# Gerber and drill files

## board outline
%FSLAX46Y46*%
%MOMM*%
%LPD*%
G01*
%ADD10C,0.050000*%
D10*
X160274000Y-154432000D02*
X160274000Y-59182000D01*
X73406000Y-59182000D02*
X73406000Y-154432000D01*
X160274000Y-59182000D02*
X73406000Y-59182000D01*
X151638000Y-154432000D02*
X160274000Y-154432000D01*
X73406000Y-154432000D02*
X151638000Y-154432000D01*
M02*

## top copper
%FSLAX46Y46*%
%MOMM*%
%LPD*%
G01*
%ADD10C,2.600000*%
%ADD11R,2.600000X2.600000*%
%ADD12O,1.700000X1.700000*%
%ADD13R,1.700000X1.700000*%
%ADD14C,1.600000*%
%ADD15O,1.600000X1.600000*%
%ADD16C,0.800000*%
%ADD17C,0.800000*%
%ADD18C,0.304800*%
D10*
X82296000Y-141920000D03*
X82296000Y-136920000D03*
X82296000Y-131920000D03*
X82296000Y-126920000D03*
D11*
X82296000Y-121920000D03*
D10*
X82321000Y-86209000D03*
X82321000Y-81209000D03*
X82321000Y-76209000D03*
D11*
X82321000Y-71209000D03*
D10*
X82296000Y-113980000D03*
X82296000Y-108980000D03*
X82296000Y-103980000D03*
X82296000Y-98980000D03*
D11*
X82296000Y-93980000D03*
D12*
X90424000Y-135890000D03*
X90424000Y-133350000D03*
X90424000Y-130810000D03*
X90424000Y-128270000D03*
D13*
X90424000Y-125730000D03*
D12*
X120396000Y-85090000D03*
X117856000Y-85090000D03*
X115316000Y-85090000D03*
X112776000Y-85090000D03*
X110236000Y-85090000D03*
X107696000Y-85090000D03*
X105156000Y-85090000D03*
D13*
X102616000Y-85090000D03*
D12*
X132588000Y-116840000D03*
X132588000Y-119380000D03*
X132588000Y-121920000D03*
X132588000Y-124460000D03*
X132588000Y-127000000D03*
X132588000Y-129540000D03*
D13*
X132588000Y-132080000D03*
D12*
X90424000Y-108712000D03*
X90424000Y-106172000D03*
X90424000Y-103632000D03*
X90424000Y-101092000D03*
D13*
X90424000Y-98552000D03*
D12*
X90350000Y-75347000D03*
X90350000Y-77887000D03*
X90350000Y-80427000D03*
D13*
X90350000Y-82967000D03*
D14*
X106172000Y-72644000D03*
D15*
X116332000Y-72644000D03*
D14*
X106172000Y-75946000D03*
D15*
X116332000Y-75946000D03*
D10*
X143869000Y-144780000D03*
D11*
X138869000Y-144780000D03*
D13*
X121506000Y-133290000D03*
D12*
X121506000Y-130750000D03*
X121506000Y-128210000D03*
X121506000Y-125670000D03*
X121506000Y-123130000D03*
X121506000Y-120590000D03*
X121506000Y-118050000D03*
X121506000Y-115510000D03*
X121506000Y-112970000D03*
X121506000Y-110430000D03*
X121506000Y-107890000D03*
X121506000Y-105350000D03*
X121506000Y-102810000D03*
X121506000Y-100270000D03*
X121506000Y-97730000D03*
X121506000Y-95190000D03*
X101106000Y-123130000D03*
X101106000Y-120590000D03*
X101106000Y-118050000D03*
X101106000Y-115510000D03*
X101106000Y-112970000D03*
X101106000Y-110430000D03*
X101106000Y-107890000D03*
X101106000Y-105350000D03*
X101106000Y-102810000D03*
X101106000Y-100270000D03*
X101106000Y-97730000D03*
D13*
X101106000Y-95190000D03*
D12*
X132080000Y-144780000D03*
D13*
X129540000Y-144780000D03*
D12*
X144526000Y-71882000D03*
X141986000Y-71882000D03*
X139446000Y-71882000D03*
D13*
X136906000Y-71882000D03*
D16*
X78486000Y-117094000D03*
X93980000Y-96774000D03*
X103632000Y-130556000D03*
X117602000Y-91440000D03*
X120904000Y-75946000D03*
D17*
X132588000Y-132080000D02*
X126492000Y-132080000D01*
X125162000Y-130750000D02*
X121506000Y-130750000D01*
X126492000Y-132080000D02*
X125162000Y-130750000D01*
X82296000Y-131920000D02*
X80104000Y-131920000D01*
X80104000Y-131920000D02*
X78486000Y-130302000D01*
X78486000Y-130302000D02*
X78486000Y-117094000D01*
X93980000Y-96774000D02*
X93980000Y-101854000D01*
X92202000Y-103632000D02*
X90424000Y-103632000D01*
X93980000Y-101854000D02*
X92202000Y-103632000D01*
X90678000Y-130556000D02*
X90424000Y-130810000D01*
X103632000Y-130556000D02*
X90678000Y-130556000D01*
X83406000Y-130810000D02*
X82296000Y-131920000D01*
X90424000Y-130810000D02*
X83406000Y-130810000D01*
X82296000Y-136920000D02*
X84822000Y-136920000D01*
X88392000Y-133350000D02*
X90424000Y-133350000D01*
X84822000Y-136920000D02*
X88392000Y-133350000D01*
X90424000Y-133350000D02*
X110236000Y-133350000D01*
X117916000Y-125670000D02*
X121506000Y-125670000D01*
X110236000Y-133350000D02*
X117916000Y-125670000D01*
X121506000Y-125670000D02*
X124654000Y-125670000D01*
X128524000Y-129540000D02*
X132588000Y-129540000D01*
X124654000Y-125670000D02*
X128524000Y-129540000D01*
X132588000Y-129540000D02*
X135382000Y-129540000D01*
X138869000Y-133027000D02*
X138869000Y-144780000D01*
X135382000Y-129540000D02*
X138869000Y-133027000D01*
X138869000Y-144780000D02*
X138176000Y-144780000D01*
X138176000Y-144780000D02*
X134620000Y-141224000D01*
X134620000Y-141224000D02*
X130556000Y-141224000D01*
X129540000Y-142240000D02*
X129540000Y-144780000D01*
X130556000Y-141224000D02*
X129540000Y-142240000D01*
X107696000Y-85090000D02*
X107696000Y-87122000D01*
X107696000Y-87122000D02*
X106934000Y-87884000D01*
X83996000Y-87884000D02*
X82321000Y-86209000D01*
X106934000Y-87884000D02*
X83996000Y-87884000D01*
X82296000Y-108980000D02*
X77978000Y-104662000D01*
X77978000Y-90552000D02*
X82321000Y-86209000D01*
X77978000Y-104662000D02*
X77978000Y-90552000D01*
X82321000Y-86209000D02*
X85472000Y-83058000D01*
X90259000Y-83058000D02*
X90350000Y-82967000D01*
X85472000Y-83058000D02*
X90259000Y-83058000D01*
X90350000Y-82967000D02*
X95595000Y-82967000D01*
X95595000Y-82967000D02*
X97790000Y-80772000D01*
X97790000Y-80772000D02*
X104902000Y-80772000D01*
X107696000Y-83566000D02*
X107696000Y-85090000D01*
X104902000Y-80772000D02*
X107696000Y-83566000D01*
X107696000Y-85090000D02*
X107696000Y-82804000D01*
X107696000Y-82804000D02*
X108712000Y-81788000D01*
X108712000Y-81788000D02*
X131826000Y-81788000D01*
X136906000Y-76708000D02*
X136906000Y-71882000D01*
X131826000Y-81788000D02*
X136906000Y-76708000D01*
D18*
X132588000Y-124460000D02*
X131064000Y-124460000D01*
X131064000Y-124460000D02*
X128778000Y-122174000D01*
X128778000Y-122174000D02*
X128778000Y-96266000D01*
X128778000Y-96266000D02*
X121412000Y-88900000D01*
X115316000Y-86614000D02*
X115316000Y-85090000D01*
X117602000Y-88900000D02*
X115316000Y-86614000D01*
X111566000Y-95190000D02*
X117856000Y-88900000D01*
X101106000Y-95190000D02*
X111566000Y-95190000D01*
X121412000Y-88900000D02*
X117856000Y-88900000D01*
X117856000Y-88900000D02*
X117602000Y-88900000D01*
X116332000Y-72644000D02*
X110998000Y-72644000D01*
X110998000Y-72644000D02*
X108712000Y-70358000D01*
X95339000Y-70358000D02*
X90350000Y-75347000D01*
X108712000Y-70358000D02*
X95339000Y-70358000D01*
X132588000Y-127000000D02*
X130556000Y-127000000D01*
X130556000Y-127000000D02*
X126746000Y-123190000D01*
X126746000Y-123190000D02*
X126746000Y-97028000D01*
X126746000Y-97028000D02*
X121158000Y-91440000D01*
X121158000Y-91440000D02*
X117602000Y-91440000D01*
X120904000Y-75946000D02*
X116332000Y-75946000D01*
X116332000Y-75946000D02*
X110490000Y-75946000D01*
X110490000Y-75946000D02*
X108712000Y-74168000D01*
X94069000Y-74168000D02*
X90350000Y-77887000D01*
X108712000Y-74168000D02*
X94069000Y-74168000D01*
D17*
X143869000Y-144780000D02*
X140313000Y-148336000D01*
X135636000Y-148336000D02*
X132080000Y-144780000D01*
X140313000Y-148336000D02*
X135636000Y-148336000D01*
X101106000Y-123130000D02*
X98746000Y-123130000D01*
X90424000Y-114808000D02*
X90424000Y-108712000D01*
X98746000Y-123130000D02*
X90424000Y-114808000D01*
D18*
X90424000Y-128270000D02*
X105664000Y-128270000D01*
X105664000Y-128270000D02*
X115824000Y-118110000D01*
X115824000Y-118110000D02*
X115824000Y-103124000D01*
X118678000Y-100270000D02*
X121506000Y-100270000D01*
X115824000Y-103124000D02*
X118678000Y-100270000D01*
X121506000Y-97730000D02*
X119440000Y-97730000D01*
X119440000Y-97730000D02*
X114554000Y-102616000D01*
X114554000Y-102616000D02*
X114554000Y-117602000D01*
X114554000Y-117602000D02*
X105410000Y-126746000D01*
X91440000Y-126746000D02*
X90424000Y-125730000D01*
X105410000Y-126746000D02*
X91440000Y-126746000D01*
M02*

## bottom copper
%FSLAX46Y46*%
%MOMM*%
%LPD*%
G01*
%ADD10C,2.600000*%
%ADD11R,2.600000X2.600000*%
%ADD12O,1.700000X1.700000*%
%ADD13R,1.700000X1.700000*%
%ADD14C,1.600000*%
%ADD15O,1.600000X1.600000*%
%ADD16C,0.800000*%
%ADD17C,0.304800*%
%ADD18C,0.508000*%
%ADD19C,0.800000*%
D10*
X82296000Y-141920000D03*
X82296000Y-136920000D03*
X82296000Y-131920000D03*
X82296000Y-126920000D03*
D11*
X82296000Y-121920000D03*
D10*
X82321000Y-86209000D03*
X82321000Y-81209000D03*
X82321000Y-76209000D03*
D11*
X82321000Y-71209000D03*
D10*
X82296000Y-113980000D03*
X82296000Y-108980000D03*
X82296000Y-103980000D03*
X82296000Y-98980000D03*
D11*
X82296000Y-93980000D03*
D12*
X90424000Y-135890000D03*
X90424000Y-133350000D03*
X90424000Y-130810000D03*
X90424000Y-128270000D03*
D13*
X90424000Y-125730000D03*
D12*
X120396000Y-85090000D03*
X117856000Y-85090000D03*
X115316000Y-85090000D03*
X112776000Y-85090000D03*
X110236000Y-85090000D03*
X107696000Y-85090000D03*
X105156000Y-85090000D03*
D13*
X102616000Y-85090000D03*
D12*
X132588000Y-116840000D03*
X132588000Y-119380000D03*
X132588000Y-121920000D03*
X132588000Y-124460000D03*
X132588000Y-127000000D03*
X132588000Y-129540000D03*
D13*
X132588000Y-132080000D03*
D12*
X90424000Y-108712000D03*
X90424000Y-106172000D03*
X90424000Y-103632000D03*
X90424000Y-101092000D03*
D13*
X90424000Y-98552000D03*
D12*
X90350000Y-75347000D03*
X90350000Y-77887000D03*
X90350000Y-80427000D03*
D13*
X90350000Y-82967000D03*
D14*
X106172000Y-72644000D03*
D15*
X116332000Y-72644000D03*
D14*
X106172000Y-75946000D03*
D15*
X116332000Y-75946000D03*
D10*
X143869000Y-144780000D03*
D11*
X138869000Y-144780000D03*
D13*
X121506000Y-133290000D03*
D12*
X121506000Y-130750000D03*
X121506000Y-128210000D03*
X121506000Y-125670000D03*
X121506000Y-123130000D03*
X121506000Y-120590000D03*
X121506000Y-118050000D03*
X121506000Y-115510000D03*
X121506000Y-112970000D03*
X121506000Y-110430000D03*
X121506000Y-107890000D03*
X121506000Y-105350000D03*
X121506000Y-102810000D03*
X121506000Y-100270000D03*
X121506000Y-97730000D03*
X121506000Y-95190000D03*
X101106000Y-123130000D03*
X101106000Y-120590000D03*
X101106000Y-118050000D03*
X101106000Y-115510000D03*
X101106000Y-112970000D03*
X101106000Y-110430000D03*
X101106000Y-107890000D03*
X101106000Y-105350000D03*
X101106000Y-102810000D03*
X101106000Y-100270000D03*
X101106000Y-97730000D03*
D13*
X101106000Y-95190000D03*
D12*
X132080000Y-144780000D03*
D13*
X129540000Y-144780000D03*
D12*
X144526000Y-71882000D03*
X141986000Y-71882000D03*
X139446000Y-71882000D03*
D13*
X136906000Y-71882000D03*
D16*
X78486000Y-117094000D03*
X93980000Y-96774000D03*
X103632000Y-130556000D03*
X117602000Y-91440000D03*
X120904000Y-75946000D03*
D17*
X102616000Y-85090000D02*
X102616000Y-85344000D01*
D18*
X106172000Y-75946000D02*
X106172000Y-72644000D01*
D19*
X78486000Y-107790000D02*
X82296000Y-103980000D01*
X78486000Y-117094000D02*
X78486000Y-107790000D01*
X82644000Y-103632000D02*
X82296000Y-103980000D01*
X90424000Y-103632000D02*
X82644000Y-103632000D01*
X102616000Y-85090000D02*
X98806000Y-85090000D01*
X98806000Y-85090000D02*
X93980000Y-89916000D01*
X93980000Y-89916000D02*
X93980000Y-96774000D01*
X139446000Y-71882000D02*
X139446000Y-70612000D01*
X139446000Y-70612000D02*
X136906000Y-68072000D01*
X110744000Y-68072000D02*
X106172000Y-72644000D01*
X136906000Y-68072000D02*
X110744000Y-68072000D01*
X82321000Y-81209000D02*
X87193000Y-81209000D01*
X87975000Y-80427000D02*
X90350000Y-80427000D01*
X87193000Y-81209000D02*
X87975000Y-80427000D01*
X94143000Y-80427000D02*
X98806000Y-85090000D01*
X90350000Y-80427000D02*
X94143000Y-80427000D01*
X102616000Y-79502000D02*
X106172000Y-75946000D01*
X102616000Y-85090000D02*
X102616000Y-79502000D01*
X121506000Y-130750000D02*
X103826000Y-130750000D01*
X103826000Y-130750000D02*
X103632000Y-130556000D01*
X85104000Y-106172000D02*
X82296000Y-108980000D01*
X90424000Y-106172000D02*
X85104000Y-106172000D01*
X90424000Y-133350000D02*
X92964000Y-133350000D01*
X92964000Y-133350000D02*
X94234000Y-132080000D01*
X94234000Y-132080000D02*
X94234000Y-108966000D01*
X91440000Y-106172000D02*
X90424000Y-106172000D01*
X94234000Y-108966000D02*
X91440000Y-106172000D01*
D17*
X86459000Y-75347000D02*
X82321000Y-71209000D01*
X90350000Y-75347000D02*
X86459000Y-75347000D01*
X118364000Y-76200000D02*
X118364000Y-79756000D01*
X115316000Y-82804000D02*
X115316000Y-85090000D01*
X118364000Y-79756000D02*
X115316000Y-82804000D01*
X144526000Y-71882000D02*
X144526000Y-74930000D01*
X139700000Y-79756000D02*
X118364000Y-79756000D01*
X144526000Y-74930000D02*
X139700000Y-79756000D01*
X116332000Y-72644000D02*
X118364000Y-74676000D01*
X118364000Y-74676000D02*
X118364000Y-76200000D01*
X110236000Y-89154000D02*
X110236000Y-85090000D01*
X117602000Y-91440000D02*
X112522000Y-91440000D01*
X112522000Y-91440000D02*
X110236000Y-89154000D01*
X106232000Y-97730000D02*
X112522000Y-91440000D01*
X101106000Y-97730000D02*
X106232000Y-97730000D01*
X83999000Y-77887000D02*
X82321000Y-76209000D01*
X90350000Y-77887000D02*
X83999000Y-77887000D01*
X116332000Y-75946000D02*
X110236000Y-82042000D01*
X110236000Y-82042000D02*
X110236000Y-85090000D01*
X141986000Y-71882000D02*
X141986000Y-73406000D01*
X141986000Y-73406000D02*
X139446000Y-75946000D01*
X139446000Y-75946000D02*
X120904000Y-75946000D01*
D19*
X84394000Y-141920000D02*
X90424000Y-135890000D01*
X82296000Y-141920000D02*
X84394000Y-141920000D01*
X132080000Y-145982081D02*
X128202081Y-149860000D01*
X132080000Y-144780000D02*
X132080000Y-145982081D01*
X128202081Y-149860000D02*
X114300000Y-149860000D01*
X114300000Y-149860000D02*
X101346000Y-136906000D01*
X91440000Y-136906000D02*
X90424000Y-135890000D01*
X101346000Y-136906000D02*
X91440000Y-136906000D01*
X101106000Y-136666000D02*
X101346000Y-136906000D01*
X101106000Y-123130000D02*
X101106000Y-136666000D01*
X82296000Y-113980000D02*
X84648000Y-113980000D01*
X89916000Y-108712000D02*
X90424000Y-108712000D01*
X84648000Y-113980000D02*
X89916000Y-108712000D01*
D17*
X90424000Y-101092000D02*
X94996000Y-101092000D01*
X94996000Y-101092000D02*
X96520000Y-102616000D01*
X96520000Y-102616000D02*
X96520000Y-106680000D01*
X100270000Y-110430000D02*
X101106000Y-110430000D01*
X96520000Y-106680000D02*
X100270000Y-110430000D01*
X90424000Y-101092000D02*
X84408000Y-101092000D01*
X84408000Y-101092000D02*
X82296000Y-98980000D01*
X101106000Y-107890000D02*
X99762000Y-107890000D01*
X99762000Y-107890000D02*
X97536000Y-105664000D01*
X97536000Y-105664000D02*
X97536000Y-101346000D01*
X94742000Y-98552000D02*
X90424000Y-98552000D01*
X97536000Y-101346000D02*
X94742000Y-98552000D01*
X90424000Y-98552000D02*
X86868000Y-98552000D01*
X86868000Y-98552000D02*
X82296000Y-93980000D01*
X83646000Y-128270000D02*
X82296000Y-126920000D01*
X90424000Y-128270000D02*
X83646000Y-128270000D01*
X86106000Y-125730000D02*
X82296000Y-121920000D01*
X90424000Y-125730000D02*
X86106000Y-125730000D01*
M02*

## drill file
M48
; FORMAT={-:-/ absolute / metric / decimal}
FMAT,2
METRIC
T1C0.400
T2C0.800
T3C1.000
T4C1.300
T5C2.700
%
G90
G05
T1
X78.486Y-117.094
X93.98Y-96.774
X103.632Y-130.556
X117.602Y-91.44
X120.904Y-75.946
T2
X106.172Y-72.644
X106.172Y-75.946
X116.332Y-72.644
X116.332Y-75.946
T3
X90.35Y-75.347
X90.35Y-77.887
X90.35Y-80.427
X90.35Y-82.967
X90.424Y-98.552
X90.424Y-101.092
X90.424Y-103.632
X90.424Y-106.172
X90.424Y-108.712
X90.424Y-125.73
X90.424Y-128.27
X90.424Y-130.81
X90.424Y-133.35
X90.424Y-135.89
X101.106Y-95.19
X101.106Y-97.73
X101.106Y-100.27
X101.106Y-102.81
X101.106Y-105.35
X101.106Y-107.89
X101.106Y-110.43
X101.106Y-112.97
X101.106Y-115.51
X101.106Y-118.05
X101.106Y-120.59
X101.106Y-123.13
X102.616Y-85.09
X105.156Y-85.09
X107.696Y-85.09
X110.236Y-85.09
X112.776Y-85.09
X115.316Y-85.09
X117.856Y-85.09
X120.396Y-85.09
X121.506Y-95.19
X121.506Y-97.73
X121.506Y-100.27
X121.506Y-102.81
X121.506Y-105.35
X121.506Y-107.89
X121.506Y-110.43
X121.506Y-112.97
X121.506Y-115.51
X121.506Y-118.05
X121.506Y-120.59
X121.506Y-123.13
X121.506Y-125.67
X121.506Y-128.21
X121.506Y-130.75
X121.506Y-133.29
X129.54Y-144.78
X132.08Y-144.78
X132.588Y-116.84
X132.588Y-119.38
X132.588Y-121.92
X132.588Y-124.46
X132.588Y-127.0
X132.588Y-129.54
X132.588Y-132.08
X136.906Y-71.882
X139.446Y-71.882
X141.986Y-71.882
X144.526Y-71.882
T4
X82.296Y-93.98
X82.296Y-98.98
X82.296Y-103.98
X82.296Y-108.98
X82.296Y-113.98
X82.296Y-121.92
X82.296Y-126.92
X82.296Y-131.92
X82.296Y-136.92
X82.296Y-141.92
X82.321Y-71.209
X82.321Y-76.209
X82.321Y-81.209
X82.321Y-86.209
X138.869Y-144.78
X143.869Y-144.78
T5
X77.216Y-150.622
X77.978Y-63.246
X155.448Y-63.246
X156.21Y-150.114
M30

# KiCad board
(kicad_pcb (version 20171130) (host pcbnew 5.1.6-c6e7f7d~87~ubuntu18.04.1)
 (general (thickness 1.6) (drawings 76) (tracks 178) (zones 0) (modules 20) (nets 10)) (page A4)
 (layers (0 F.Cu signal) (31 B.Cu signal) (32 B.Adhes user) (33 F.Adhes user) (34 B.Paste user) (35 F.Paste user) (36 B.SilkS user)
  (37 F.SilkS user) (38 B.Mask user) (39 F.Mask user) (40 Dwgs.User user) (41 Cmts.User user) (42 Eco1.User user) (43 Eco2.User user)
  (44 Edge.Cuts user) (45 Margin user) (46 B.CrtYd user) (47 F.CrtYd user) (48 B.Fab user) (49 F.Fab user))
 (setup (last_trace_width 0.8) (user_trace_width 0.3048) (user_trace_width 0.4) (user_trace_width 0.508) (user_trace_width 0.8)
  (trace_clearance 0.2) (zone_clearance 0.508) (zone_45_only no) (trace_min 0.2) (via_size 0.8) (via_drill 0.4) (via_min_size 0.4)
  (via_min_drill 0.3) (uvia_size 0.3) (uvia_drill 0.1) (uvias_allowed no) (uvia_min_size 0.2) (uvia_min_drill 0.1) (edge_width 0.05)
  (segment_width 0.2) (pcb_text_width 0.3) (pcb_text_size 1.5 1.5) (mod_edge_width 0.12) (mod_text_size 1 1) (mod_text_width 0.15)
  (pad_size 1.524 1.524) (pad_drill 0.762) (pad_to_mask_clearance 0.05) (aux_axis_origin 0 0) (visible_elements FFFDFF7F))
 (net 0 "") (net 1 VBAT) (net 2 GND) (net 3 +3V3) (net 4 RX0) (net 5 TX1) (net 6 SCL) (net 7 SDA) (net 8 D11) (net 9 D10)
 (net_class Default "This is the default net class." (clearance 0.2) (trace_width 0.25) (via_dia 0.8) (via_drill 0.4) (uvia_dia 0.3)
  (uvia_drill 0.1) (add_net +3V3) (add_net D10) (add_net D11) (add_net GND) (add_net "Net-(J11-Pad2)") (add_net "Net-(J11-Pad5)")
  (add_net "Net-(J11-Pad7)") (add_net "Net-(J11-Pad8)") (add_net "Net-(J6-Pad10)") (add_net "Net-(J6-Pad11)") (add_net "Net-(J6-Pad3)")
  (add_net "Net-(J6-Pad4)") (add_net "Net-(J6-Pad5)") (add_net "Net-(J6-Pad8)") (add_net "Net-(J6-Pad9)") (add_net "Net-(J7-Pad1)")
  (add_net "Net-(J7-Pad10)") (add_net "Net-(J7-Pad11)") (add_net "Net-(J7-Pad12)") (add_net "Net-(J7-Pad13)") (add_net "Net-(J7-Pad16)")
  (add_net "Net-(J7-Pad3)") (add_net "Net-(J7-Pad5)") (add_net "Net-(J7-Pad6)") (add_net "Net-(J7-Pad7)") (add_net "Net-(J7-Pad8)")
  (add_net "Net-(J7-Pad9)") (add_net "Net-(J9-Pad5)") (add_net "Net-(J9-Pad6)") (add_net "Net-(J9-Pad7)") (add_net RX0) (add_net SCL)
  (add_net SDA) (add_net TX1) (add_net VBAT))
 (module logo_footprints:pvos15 (layer F.Cu) (at 89.408 148.844)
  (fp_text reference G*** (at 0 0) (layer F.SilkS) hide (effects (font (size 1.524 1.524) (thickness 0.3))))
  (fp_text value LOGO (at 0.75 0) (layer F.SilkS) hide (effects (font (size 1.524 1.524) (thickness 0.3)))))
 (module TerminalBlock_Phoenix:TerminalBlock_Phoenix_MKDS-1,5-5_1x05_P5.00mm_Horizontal (layer F.Cu) (at 82.296 121.92 270)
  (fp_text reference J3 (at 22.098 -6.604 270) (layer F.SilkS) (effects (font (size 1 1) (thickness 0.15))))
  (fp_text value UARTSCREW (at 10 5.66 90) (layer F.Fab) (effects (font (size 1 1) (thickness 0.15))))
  (pad 5 thru_hole circle (at 20 0 270) (size 2.6 2.6) (drill 1.3) (layers *.Cu *.Mask) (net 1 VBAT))
  (pad 4 thru_hole circle (at 15 0 270) (size 2.6 2.6) (drill 1.3) (layers *.Cu *.Mask) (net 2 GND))
  (pad 3 thru_hole circle (at 10 0 270) (size 2.6 2.6) (drill 1.3) (layers *.Cu *.Mask) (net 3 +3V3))
  (pad 2 thru_hole circle (at 5 0 270) (size 2.6 2.6) (drill 1.3) (layers *.Cu *.Mask) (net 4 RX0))
  (pad 1 thru_hole rect (at 0 0 270) (size 2.6 2.6) (drill 1.3) (layers *.Cu *.Mask) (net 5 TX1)))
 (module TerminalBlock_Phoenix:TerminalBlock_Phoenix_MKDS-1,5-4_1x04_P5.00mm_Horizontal (layer F.Cu) (at 82.321 71.209 270)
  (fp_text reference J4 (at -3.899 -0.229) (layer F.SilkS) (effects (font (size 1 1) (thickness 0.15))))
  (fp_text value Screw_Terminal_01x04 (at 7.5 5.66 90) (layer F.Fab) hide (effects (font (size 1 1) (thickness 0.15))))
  (pad 4 thru_hole circle (at 15 0 270) (size 2.6 2.6) (drill 1.3) (layers *.Cu *.Mask) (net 2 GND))
  (pad 3 thru_hole circle (at 10 0 270) (size 2.6 2.6) (drill 1.3) (layers *.Cu *.Mask) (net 3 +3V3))
  (pad 2 thru_hole circle (at 5 0 270) (size 2.6 2.6) (drill 1.3) (layers *.Cu *.Mask) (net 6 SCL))
  (pad 1 thru_hole rect (at 0 0 270) (size 2.6 2.6) (drill 1.3) (layers *.Cu *.Mask) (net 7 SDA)))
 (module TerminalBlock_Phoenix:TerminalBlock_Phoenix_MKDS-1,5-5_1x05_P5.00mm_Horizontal (layer F.Cu) (at 82.296 93.98 270)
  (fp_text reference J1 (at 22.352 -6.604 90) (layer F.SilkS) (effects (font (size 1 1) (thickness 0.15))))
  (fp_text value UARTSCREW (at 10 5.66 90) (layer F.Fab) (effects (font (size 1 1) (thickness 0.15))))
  (pad 5 thru_hole circle (at 20 0 270) (size 2.6 2.6) (drill 1.3) (layers *.Cu *.Mask) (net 1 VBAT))
  (pad 4 thru_hole circle (at 15 0 270) (size 2.6 2.6) (drill 1.3) (layers *.Cu *.Mask) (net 2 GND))
  (pad 3 thru_hole circle (at 10 0 270) (size 2.6 2.6) (drill 1.3) (layers *.Cu *.Mask) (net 3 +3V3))
  (pad 2 thru_hole circle (at 5 0 270) (size 2.6 2.6) (drill 1.3) (layers *.Cu *.Mask) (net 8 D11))
  (pad 1 thru_hole rect (at 0 0 270) (size 2.6 2.6) (drill 1.3) (layers *.Cu *.Mask) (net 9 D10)))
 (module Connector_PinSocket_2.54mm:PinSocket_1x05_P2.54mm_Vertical (layer F.Cu) (at 90.424 125.73)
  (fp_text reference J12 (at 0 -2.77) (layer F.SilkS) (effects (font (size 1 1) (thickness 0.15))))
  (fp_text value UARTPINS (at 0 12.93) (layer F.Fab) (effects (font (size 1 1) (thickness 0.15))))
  (pad 5 thru_hole oval (at 0 10.16) (size 1.7 1.7) (drill 1) (layers *.Cu *.Mask) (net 1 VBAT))
  (pad 4 thru_hole oval (at 0 7.62) (size 1.7 1.7) (drill 1) (layers *.Cu *.Mask) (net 2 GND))
  (pad 3 thru_hole oval (at 0 5.08) (size 1.7 1.7) (drill 1) (layers *.Cu *.Mask) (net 3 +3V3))
  (pad 2 thru_hole oval (at 0 2.54) (size 1.7 1.7) (drill 1) (layers *.Cu *.Mask) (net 4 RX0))
  (pad 1 thru_hole rect (at 0 0) (size 1.7 1.7) (drill 1) (layers *.Cu *.Mask) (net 5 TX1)))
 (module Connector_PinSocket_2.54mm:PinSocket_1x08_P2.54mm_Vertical (layer F.Cu) (at 102.616 85.09 90)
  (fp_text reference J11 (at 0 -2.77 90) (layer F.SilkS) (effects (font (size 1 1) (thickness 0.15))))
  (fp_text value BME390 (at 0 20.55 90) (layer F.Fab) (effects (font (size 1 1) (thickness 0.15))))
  (pad 8 thru_hole oval (at 0 17.78 90) (size 1.7 1.7) (drill 1) (layers *.Cu *.Mask))
  (pad 7 thru_hole oval (at 0 15.24 90) (size 1.7 1.7) (drill 1) (layers *.Cu *.Mask))
  (pad 6 thru_hole oval (at 0 12.7 90) (size 1.7 1.7) (drill 1) (layers *.Cu *.Mask) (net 7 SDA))
  (pad 5 thru_hole oval (at 0 10.16 90) (size 1.7 1.7) (drill 1) (layers *.Cu *.Mask))
  (pad 4 thru_hole oval (at 0 7.62 90) (size 1.7 1.7) (drill 1) (layers *.Cu *.Mask) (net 6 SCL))
  (pad 3 thru_hole oval (at 0 5.08 90) (size 1.7 1.7) (drill 1) (layers *.Cu *.Mask) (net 2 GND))
  (pad 2 thru_hole oval (at 0 2.54 90) (size 1.7 1.7) (drill 1) (layers *.Cu *.Mask))
  (pad 1 thru_hole rect (at 0 0 90) (size 1.7 1.7) (drill 1) (layers *.Cu *.Mask) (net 3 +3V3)))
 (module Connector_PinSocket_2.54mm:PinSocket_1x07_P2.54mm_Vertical (layer F.Cu) (at 132.588 132.08 180)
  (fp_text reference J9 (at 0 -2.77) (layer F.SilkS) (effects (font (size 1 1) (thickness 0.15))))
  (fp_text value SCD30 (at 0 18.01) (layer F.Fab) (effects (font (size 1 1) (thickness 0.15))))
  (pad 7 thru_hole oval (at 0 15.24 180) (size 1.7 1.7) (drill 1) (layers *.Cu *.Mask))
  (pad 6 thru_hole oval (at 0 12.7 180) (size 1.7 1.7) (drill 1) (layers *.Cu *.Mask))
  (pad 5 thru_hole oval (at 0 10.16 180) (size 1.7 1.7) (drill 1) (layers *.Cu *.Mask))
  (pad 4 thru_hole oval (at 0 7.62 180) (size 1.7 1.7) (drill 1) (layers *.Cu *.Mask) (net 7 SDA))
  (pad 3 thru_hole oval (at 0 5.08 180) (size 1.7 1.7) (drill 1) (layers *.Cu *.Mask) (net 6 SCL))
  (pad 2 thru_hole oval (at 0 2.54 180) (size 1.7 1.7) (drill 1) (layers *.Cu *.Mask) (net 2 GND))
  (pad 1 thru_hole rect (at 0 0 180) (size 1.7 1.7) (drill 1) (layers *.Cu *.Mask) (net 3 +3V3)))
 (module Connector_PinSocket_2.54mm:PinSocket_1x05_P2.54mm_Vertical (layer F.Cu) (at 90.424 98.552)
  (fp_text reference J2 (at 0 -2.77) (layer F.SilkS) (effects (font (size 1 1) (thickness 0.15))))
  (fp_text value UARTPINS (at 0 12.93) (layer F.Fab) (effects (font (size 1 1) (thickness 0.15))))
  (pad 5 thru_hole oval (at 0 10.16) (size 1.7 1.7) (drill 1) (layers *.Cu *.Mask) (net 1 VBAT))
  (pad 4 thru_hole oval (at 0 7.62) (size 1.7 1.7) (drill 1) (layers *.Cu *.Mask) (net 2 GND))
  (pad 3 thru_hole oval (at 0 5.08) (size 1.7 1.7) (drill 1) (layers *.Cu *.Mask) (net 3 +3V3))
  (pad 2 thru_hole oval (at 0 2.54) (size 1.7 1.7) (drill 1) (layers *.Cu *.Mask) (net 8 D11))
  (pad 1 thru_hole rect (at 0 0) (size 1.7 1.7) (drill 1) (layers *.Cu *.Mask) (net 9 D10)))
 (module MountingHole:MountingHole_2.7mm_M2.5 (layer F.Cu) (at 156.21 150.114)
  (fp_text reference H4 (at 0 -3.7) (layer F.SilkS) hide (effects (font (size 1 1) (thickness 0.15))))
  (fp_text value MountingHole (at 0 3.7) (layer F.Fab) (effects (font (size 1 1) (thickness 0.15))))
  (pad 1 np_thru_hole circle (at 0 0) (size 2.7 2.7) (drill 2.7) (layers *.Cu *.Mask)))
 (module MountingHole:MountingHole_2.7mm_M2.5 (layer F.Cu) (at 77.216 150.622)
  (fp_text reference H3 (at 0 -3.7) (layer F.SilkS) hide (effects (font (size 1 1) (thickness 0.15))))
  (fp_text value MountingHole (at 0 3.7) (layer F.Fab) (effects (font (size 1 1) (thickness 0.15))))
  (pad 1 np_thru_hole circle (at 0 0) (size 2.7 2.7) (drill 2.7) (layers *.Cu *.Mask)))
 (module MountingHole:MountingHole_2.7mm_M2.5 (layer F.Cu) (at 155.448 63.246)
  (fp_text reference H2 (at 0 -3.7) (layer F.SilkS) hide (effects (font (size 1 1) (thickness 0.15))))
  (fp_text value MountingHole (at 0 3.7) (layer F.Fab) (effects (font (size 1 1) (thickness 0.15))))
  (pad 1 np_thru_hole circle (at 0 0) (size 2.7 2.7) (drill 2.7) (layers *.Cu *.Mask)))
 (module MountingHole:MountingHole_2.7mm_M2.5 (layer F.Cu) (at 77.978 63.246)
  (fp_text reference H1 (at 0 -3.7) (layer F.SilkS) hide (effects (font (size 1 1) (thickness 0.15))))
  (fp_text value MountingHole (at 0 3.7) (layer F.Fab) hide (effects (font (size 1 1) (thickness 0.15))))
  (pad 1 np_thru_hole circle (at 0 0) (size 2.7 2.7) (drill 2.7) (layers *.Cu *.Mask)))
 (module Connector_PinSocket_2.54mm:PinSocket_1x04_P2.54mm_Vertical (layer F.Cu) (at 90.35 82.967 180)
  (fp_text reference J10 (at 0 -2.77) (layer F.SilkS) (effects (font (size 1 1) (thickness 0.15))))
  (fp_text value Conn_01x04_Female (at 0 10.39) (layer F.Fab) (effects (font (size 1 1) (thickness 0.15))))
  (pad 4 thru_hole oval (at 0 7.62 180) (size 1.7 1.7) (drill 1) (layers *.Cu *.Mask) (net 7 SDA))
  (pad 3 thru_hole oval (at 0 5.08 180) (size 1.7 1.7) (drill 1) (layers *.Cu *.Mask) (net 6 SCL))
  (pad 2 thru_hole oval (at 0 2.54 180) (size 1.7 1.7) (drill 1) (layers *.Cu *.Mask) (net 3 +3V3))
  (pad 1 thru_hole rect (at 0 0 180) (size 1.7 1.7) (drill 1) (layers *.Cu *.Mask) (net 2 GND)))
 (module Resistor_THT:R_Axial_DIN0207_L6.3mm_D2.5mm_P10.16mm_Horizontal (layer F.Cu) (at 106.172 72.644)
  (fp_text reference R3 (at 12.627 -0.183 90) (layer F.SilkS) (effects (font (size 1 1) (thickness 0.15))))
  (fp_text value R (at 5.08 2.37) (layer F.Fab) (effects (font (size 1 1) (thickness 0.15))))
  (pad 1 thru_hole circle (at 0 0) (size 1.6 1.6) (drill 0.8) (layers *.Cu *.Mask) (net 3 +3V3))
  (pad 2 thru_hole oval (at 10.16 0) (size 1.6 1.6) (drill 0.8) (layers *.Cu *.Mask) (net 7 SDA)))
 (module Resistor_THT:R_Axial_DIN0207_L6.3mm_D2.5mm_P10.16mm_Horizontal (layer F.Cu) (at 106.172 75.946)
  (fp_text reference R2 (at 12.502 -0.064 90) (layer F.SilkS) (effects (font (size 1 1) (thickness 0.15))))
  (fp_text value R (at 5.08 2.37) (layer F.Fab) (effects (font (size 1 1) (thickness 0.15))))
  (pad 1 thru_hole circle (at 0 0) (size 1.6 1.6) (drill 0.8) (layers *.Cu *.Mask) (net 3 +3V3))
  (pad 2 thru_hole oval (at 10.16 0) (size 1.6 1.6) (drill 0.8) (layers *.Cu *.Mask) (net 6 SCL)))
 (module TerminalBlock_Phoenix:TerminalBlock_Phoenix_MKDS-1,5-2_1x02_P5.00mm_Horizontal (layer F.Cu) (at 138.869 144.78)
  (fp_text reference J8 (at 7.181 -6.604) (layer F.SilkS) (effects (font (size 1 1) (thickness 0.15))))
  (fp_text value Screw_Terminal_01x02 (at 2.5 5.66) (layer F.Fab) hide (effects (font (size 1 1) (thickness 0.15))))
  (pad 2 thru_hole circle (at 5 0) (size 2.6 2.6) (drill 1.3) (layers *.Cu *.Mask) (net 1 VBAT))
  (pad 1 thru_hole rect (at 0 0) (size 2.6 2.6) (drill 1.3) (layers *.Cu *.Mask) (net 2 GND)))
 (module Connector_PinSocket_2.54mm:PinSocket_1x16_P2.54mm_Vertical (layer F.Cu) (at 121.506 133.29 180)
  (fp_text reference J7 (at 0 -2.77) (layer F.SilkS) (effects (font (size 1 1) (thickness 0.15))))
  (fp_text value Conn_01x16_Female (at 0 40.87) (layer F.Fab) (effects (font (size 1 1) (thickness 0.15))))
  (pad 1 thru_hole rect (at 0 0 180) (size 1.7 1.7) (drill 1) (layers *.Cu *.Mask))
  (pad 2 thru_hole oval (at 0 2.54 180) (size 1.7 1.7) (drill 1) (layers *.Cu *.Mask) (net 3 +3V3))
  (pad 3 thru_hole oval (at 0 5.08 180) (size 1.7 1.7) (drill 1) (layers *.Cu *.Mask))
  (pad 4 thru_hole oval (at 0 7.62 180) (size 1.7 1.7) (drill 1) (layers *.Cu *.Mask) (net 2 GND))
  (pad 5 thru_hole oval (at 0 10.16 180) (size 1.7 1.7) (drill 1) (layers *.Cu *.Mask))
  (pad 6 thru_hole oval (at 0 12.7 180) (size 1.7 1.7) (drill 1) (layers *.Cu *.Mask))
  (pad 7 thru_hole oval (at 0 15.24 180) (size 1.7 1.7) (drill 1) (layers *.Cu *.Mask))
  (pad 8 thru_hole oval (at 0 17.78 180) (size 1.7 1.7) (drill 1) (layers *.Cu *.Mask))
  (pad 9 thru_hole oval (at 0 20.32 180) (size 1.7 1.7) (drill 1) (layers *.Cu *.Mask))
  (pad 10 thru_hole oval (at 0 22.86 180) (size 1.7 1.7) (drill 1) (layers *.Cu *.Mask))
  (pad 11 thru_hole oval (at 0 25.4 180) (size 1.7 1.7) (drill 1) (layers *.Cu *.Mask))
  (pad 12 thru_hole oval (at 0 27.94 180) (size 1.7 1.7) (drill 1) (layers *.Cu *.Mask))
  (pad 13 thru_hole oval (at 0 30.48 180) (size 1.7 1.7) (drill 1) (layers *.Cu *.Mask))
  (pad 14 thru_hole oval (at 0 33.02 180) (size 1.7 1.7) (drill 1) (layers *.Cu *.Mask) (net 4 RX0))
  (pad 15 thru_hole oval (at 0 35.56 180) (size 1.7 1.7) (drill 1) (layers *.Cu *.Mask) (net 5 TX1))
  (pad 16 thru_hole oval (at 0 38.1 180) (size 1.7 1.7) (drill 1) (layers *.Cu *.Mask)))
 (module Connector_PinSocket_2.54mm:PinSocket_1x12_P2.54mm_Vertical (layer F.Cu) (at 101.106 95.19)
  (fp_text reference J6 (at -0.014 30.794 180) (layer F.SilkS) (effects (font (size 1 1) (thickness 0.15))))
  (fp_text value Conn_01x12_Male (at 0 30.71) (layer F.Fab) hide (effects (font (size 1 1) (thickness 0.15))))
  (pad 12 thru_hole oval (at 0 27.94) (size 1.7 1.7) (drill 1) (layers *.Cu *.Mask) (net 1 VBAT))
  (pad 11 thru_hole oval (at 0 25.4) (size 1.7 1.7) (drill 1) (layers *.Cu *.Mask))
  (pad 10 thru_hole oval (at 0 22.86) (size 1.7 1.7) (drill 1) (layers *.Cu *.Mask))
  (pad 9 thru_hole oval (at 0 20.32) (size 1.7 1.7) (drill 1) (layers *.Cu *.Mask))
  (pad 8 thru_hole oval (at 0 17.78) (size 1.7 1.7) (drill 1) (layers *.Cu *.Mask))
  (pad 7 thru_hole oval (at 0 15.24) (size 1.7 1.7) (drill 1) (layers *.Cu *.Mask) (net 8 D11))
  (pad 6 thru_hole oval (at 0 12.7) (size 1.7 1.7) (drill 1) (layers *.Cu *.Mask) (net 9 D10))
  (pad 5 thru_hole oval (at 0 10.16) (size 1.7 1.7) (drill 1) (layers *.Cu *.Mask))
  (pad 4 thru_hole oval (at 0 7.62) (size 1.7 1.7) (drill 1) (layers *.Cu *.Mask))
  (pad 3 thru_hole oval (at 0 5.08) (size 1.7 1.7) (drill 1) (layers *.Cu *.Mask))
  (pad 2 thru_hole oval (at 0 2.54) (size 1.7 1.7) (drill 1) (layers *.Cu *.Mask) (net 6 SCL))
  (pad 1 thru_hole rect (at 0 0) (size 1.7 1.7) (drill 1) (layers *.Cu *.Mask) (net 7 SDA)))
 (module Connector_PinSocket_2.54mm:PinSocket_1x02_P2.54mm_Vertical (layer F.Cu) (at 129.54 144.78 90)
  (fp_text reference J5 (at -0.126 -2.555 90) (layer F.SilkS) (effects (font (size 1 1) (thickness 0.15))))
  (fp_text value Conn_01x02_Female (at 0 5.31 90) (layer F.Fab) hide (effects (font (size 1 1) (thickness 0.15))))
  (pad 2 thru_hole oval (at 0 2.54 90) (size 1.7 1.7) (drill 1) (layers *.Cu *.Mask) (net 1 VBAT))
  (pad 1 thru_hole rect (at 0 0 90) (size 1.7 1.7) (drill 1) (layers *.Cu *.Mask) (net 2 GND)))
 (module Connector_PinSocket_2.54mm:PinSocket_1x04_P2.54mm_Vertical (layer F.Cu) (at 136.906 71.882 90)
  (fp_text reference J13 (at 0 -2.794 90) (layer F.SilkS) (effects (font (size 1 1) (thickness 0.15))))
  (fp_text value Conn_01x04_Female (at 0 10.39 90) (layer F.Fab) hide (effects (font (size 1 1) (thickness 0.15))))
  (pad 4 thru_hole oval (at 0 7.62 90) (size 1.7 1.7) (drill 1) (layers *.Cu *.Mask) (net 7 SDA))
  (pad 3 thru_hole oval (at 0 5.08 90) (size 1.7 1.7) (drill 1) (layers *.Cu *.Mask) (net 6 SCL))
  (pad 2 thru_hole oval (at 0 2.54 90) (size 1.7 1.7) (drill 1) (layers *.Cu *.Mask) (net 3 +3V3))
  (pad 1 thru_hole rect (at 0 0 90) (size 1.7 1.7) (drill 1) (layers *.Cu *.Mask) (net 2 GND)))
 (gr_line (start 160.274 154.432) (end 160.274 59.182) (layer Edge.Cuts) (width 0.05))
 (gr_line (start 73.406 59.182) (end 73.406 154.432) (layer Edge.Cuts) (width 0.05))
 (gr_line (start 160.274 59.182) (end 73.406 59.182) (layer Edge.Cuts) (width 0.05))
 (gr_line (start 151.638 154.432) (end 160.274 154.432) (layer Edge.Cuts) (width 0.05))
 (gr_line (start 73.406 154.432) (end 151.638 154.432) (layer Edge.Cuts) (width 0.05))
 (segment (start 102.616 85.09) (end 102.616 85.344) (width 0.3048) (layer B.Cu) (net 3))
 (segment (start 106.172 75.946) (end 106.172 72.644) (width 0.508) (layer B.Cu) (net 3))
 (segment (start 132.588 132.08) (end 126.492 132.08) (width 0.8) (layer F.Cu) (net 3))
 (segment (start 125.162 130.75) (end 121.506 130.75) (width 0.8) (layer F.Cu) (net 3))
 (segment (start 126.492 132.08) (end 125.162 130.75) (width 0.8) (layer F.Cu) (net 3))
 (segment (start 82.296 131.92) (end 80.104 131.92) (width 0.8) (layer F.Cu) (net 3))
 (segment (start 80.104 131.92) (end 78.486 130.302) (width 0.8) (layer F.Cu) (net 3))
 (via (at 78.486 117.094) (size 0.8) (drill 0.4) (layers F.Cu B.Cu) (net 3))
 (segment (start 78.486 130.302) (end 78.486 117.094) (width 0.8) (layer F.Cu) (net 3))
 (segment (start 78.486 107.79) (end 82.296 103.98) (width 0.8) (layer B.Cu) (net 3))
 (segment (start 78.486 117.094) (end 78.486 107.79) (width 0.8) (layer B.Cu) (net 3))
 (segment (start 82.644 103.632) (end 82.296 103.98) (width 0.8) (layer B.Cu) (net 3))
 (segment (start 90.424 103.632) (end 82.644 103.632) (width 0.8) (layer B.Cu) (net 3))
 (segment (start 102.616 85.09) (end 98.806 85.09) (width 0.8) (layer B.Cu) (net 3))
 (via (at 93.98 96.774) (size 0.8) (drill 0.4) (layers F.Cu B.Cu) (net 3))
 (segment (start 98.806 85.09) (end 93.98 89.916) (width 0.8) (layer B.Cu) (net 3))
 (segment (start 93.98 89.916) (end 93.98 96.774) (width 0.8) (layer B.Cu) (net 3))
 (segment (start 93.98 96.774) (end 93.98 101.854) (width 0.8) (layer F.Cu) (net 3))
 (segment (start 92.202 103.632) (end 90.424 103.632) (width 0.8) (layer F.Cu) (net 3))
 (segment (start 93.98 101.854) (end 92.202 103.632) (width 0.8) (layer F.Cu) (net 3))
 (segment (start 139.446 71.882) (end 139.446 70.612) (width 0.8) (layer B.Cu) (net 3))
 (segment (start 139.446 70.612) (end 136.906 68.072) (width 0.8) (layer B.Cu) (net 3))
 (segment (start 110.744 68.072) (end 106.172 72.644) (width 0.8) (layer B.Cu) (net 3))
 (segment (start 136.906 68.072) (end 110.744 68.072) (width 0.8) (layer B.Cu) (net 3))
 (segment (start 82.321 81.209) (end 87.193 81.209) (width 0.8) (layer B.Cu) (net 3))
 (segment (start 87.975 80.427) (end 90.35 80.427) (width 0.8) (layer B.Cu) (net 3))
 (segment (start 87.193 81.209) (end 87.975 80.427) (width 0.8) (layer B.Cu) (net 3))
 (segment (start 94.143 80.427) (end 98.806 85.09) (width 0.8) (layer B.Cu) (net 3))
 (segment (start 90.35 80.427) (end 94.143 80.427) (width 0.8) (layer B.Cu) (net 3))
 (segment (start 102.616 79.502) (end 106.172 75.946) (width 0.8) (layer B.Cu) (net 3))
 (segment (start 102.616 85.09) (end 102.616 79.502) (width 0.8) (layer B.Cu) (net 3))
 (via (at 103.632 130.556) (size 0.8) (drill 0.4) (layers F.Cu B.Cu) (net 3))
 (segment (start 121.506 130.75) (end 103.826 130.75) (width 0.8) (layer B.Cu) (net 3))
 (segment (start 103.826 130.75) (end 103.632 130.556) (width 0.8) (layer B.Cu) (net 3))
 (segment (start 90.678 130.556) (end 90.424 130.81) (width 0.8) (layer F.Cu) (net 3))
 (segment (start 103.632 130.556) (end 90.678 130.556) (width 0.8) (layer F.Cu) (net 3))
 (segment (start 83.406 130.81) (end 82.296 131.92) (width 0.8) (layer F.Cu) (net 3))
 (segment (start 90.424 130.81) (end 83.406 130.81) (width 0.8) (layer F.Cu) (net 3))
 (segment (start 82.296 136.92) (end 84.822 136.92) (width 0.8) (layer F.Cu) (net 2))
 (segment (start 88.392 133.35) (end 90.424 133.35) (width 0.8) (layer F.Cu) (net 2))
 (segment (start 84.822 136.92) (end 88.392 133.35) (width 0.8) (layer F.Cu) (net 2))
 (segment (start 90.424 133.35) (end 110.236 133.35) (width 0.8) (layer F.Cu) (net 2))
 (segment (start 117.916 125.67) (end 121.506 125.67) (width 0.8) (layer F.Cu) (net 2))
 (segment (start 110.236 133.35) (end 117.916 125.67) (width 0.8) (layer F.Cu) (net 2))
 (segment (start 121.506 125.67) (end 124.654 125.67) (width 0.8) (layer F.Cu) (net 2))
 (segment (start 128.524 129.54) (end 132.588 129.54) (width 0.8) (layer F.Cu) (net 2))
 (segment (start 124.654 125.67) (end 128.524 129.54) (width 0.8) (layer F.Cu) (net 2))
 (segment (start 132.588 129.54) (end 135.382 129.54) (width 0.8) (layer F.Cu) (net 2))
 (segment (start 138.869 133.027) (end 138.869 144.78) (width 0.8) (layer F.Cu) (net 2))
 (segment (start 135.382 129.54) (end 138.869 133.027) (width 0.8) (layer F.Cu) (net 2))
 (segment (start 138.869 144.78) (end 138.176 144.78) (width 0.8) (layer F.Cu) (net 2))
 (segment (start 138.176 144.78) (end 134.62 141.224) (width 0.8) (layer F.Cu) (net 2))
 (segment (start 134.62 141.224) (end 130.556 141.224) (width 0.8) (layer F.Cu) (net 2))
 (segment (start 129.54 142.24) (end 129.54 144.78) (width 0.8) (layer F.Cu) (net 2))
 (segment (start 130.556 141.224) (end 129.54 142.24) (width 0.8) (layer F.Cu) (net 2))
 (segment (start 85.104 106.172) (end 82.296 108.98) (width 0.8) (layer B.Cu) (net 2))
 (segment (start 90.424 106.172) (end 85.104 106.172) (width 0.8) (layer B.Cu) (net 2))
 (segment (start 107.696 85.09) (end 107.696 87.122) (width 0.8) (layer F.Cu) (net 2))
 (segment (start 107.696 87.122) (end 106.934 87.884) (width 0.8) (layer F.Cu) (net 2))
 (segment (start 83.996 87.884) (end 82.321 86.209) (width 0.8) (layer F.Cu) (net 2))
 (segment (start 106.934 87.884) (end 83.996 87.884) (width 0.8) (layer F.Cu) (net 2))
 (segment (start 82.296 108.98) (end 77.978 104.662) (width 0.8) (layer F.Cu) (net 2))
 (segment (start 77.978 90.552) (end 82.321 86.209) (width 0.8) (layer F.Cu) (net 2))
 (segment (start 77.978 104.662) (end 77.978 90.552) (width 0.8) (layer F.Cu) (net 2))
 (segment (start 82.321 86.209) (end 85.472 83.058) (width 0.8) (layer F.Cu) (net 2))
 (segment (start 90.259 83.058) (end 90.35 82.967) (width 0.8) (layer F.Cu) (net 2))
 (segment (start 85.472 83.058) (end 90.259 83.058) (width 0.8) (layer F.Cu) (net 2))
 (segment (start 90.35 82.967) (end 95.595 82.967) (width 0.8) (layer F.Cu) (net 2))
 (segment (start 95.595 82.967) (end 97.79 80.772) (width 0.8) (layer F.Cu) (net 2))
 (segment (start 97.79 80.772) (end 104.902 80.772) (width 0.8) (layer F.Cu) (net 2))
 (segment (start 107.696 83.566) (end 107.696 85.09) (width 0.8) (layer F.Cu) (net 2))
 (segment (start 104.902 80.772) (end 107.696 83.566) (width 0.8) (layer F.Cu) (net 2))
 (segment (start 107.696 85.09) (end 107.696 82.804) (width 0.8) (layer F.Cu) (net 2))
 (segment (start 107.696 82.804) (end 108.712 81.788) (width 0.8) (layer F.Cu) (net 2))
 (segment (start 108.712 81.788) (end 131.826 81.788) (width 0.8) (layer F.Cu) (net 2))
 (segment (start 136.906 76.708) (end 136.906 71.882) (width 0.8) (layer F.Cu) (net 2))
 (segment (start 131.826 81.788) (end 136.906 76.708) (width 0.8) (layer F.Cu) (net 2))
 (segment (start 90.424 133.35) (end 92.964 133.35) (width 0.8) (layer B.Cu) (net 2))
 (segment (start 92.964 133.35) (end 94.234 132.08) (width 0.8) (layer B.Cu) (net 2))
 (segment (start 94.234 132.08) (end 94.234 108.966) (width 0.8) (layer B.Cu) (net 2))
 (segment (start 91.44 106.172) (end 90.424 106.172) (width 0.8) (layer B.Cu) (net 2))
 (segment (start 94.234 108.966) (end 91.44 106.172) (width 0.8) (layer B.Cu) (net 2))
 (segment (start 132.588 124.46) (end 131.064 124.46) (width 0.3048) (layer F.Cu) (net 7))
 (segment (start 131.064 124.46) (end 128.778 122.174) (width 0.3048) (layer F.Cu) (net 7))
 (segment (start 128.778 122.174) (end 128.778 96.266) (width 0.3048) (layer F.Cu) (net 7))
 (segment (start 128.778 96.266) (end 121.412 88.9) (width 0.3048) (layer F.Cu) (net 7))
 (segment (start 115.316 86.614) (end 115.316 85.09) (width 0.3048) (layer F.Cu) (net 7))
 (segment (start 117.602 88.9) (end 115.316 86.614) (width 0.3048) (layer F.Cu) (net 7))
 (segment (start 111.566 95.19) (end 117.856 88.9) (width 0.3048) (layer F.Cu) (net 7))
 (segment (start 101.106 95.19) (end 111.566 95.19) (width 0.3048) (layer F.Cu) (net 7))
 (segment (start 121.412 88.9) (end 117.856 88.9) (width 0.3048) (layer F.Cu) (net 7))
 (segment (start 117.856 88.9) (end 117.602 88.9) (width 0.3048) (layer F.Cu) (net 7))
 (segment (start 86.459 75.347) (end 82.321 71.209) (width 0.3048) (layer B.Cu) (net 7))
 (segment (start 90.35 75.347) (end 86.459 75.347) (width 0.3048) (layer B.Cu) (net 7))
 (segment (start 118.364 76.2) (end 118.364 79.756) (width 0.3048) (layer B.Cu) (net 7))
 (segment (start 115.316 82.804) (end 115.316 85.09) (width 0.3048) (layer B.Cu) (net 7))
 (segment (start 118.364 79.756) (end 115.316 82.804) (width 0.3048) (layer B.Cu) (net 7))
 (segment (start 144.526 71.882) (end 144.526 74.93) (width 0.3048) (layer B.Cu) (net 7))
 (segment (start 139.7 79.756) (end 118.364 79.756) (width 0.3048) (layer B.Cu) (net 7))
 (segment (start 144.526 74.93) (end 139.7 79.756) (width 0.3048) (layer B.Cu) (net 7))
 (segment (start 116.332 72.644) (end 118.364 74.676) (width 0.3048) (layer B.Cu) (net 7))
 (segment (start 118.364 74.676) (end 118.364 76.2) (width 0.3048) (layer B.Cu) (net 7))
 (segment (start 116.332 72.644) (end 110.998 72.644) (width 0.3048) (layer F.Cu) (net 7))
 (segment (start 110.998 72.644) (end 108.712 70.358) (width 0.3048) (layer F.Cu) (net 7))
 (segment (start 95.339 70.358) (end 90.35 75.347) (width 0.3048) (layer F.Cu) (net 7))
 (segment (start 108.712 70.358) (end 95.339 70.358) (width 0.3048) (layer F.Cu) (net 7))
 (segment (start 132.588 127) (end 130.556 127) (width 0.3048) (layer F.Cu) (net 6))
 (segment (start 130.556 127) (end 126.746 123.19) (width 0.3048) (layer F.Cu) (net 6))
 (segment (start 126.746 123.19) (end 126.746 97.028) (width 0.3048) (layer F.Cu) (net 6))
 (via (at 117.602 91.44) (size 0.8) (drill 0.4) (layers F.Cu B.Cu) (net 6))
 (segment (start 126.746 97.028) (end 121.158 91.44) (width 0.3048) (layer F.Cu) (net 6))
 (segment (start 121.158 91.44) (end 117.602 91.44) (width 0.3048) (layer F.Cu) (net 6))
 (segment (start 110.236 89.154) (end 110.236 85.09) (width 0.3048) (layer B.Cu) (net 6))
 (segment (start 117.602 91.44) (end 112.522 91.44) (width 0.3048) (layer B.Cu) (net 6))
 (segment (start 112.522 91.44) (end 110.236 89.154) (width 0.3048) (layer B.Cu) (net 6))
 (segment (start 106.232 97.73) (end 112.522 91.44) (width 0.3048) (layer B.Cu) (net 6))
 (segment (start 101.106 97.73) (end 106.232 97.73) (width 0.3048) (layer B.Cu) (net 6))
 (segment (start 83.999 77.887) (end 82.321 76.209) (width 0.3048) (layer B.Cu) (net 6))
 (segment (start 90.35 77.887) (end 83.999 77.887) (width 0.3048) (layer B.Cu) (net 6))
 (segment (start 116.332 75.946) (end 110.236 82.042) (width 0.3048) (layer B.Cu) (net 6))
 (segment (start 110.236 82.042) (end 110.236 85.09) (width 0.3048) (layer B.Cu) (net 6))
 (segment (start 141.986 71.882) (end 141.986 73.406) (width 0.3048) (layer B.Cu) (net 6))
 (via (at 120.904 75.946) (size 0.8) (drill 0.4) (layers F.Cu B.Cu) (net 6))
 (segment (start 141.986 73.406) (end 139.446 75.946) (width 0.3048) (layer B.Cu) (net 6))
 (segment (start 139.446 75.946) (end 120.904 75.946) (width 0.3048) (layer B.Cu) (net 6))
 (segment (start 120.904 75.946) (end 116.332 75.946) (width 0.3048) (layer F.Cu) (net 6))
 (segment (start 116.332 75.946) (end 110.49 75.946) (width 0.3048) (layer F.Cu) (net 6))
 (segment (start 110.49 75.946) (end 108.712 74.168) (width 0.3048) (layer F.Cu) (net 6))
 (segment (start 94.069 74.168) (end 90.35 77.887) (width 0.3048) (layer F.Cu) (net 6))
 (segment (start 108.712 74.168) (end 94.069 74.168) (width 0.3048) (layer F.Cu) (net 6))
 (segment (start 84.394 141.92) (end 90.424 135.89) (width 0.8) (layer B.Cu) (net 1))
 (segment (start 82.296 141.92) (end 84.394 141.92) (width 0.8) (layer B.Cu) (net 1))
 (segment (start 143.869 144.78) (end 140.313 148.336) (width 0.8) (layer F.Cu) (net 1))
 (segment (start 135.636 148.336) (end 132.08 144.78) (width 0.8) (layer F.Cu) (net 1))
 (segment (start 140.313 148.336) (end 135.636 148.336) (width 0.8) (layer F.Cu) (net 1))
 (segment (start 132.08 145.982081) (end 128.202081 149.86) (width 0.8) (layer B.Cu) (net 1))
 (segment (start 132.08 144.78) (end 132.08 145.982081) (width 0.8) (layer B.Cu) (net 1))
 (segment (start 128.202081 149.86) (end 114.3 149.86) (width 0.8) (layer B.Cu) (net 1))
 (segment (start 114.3 149.86) (end 101.346 136.906) (width 0.8) (layer B.Cu) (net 1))
 (segment (start 91.44 136.906) (end 90.424 135.89) (width 0.8) (layer B.Cu) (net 1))
 (segment (start 101.346 136.906) (end 91.44 136.906) (width 0.8) (layer B.Cu) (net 1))
 (segment (start 101.106 136.666) (end 101.346 136.906) (width 0.8) (layer B.Cu) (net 1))
 (segment (start 101.106 123.13) (end 101.106 136.666) (width 0.8) (layer B.Cu) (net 1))
 (segment (start 82.296 113.98) (end 84.648 113.98) (width 0.8) (layer B.Cu) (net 1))
 (segment (start 89.916 108.712) (end 90.424 108.712) (width 0.8) (layer B.Cu) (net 1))
 (segment (start 84.648 113.98) (end 89.916 108.712) (width 0.8) (layer B.Cu) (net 1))
 (segment (start 101.106 123.13) (end 98.746 123.13) (width 0.8) (layer F.Cu) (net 1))
 (segment (start 90.424 114.808) (end 90.424 108.712) (width 0.8) (layer F.Cu) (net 1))
 (segment (start 98.746 123.13) (end 90.424 114.808) (width 0.8) (layer F.Cu) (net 1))
 (segment (start 90.424 101.092) (end 94.996 101.092) (width 0.3048) (layer B.Cu) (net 8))
 (segment (start 94.996 101.092) (end 96.52 102.616) (width 0.3048) (layer B.Cu) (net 8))
 (segment (start 96.52 102.616) (end 96.52 106.68) (width 0.3048) (layer B.Cu) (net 8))
 (segment (start 100.27 110.43) (end 101.106 110.43) (width 0.3048) (layer B.Cu) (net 8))
 (segment (start 96.52 106.68) (end 100.27 110.43) (width 0.3048) (layer B.Cu) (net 8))
 (segment (start 90.424 101.092) (end 84.408 101.092) (width 0.3048) (layer B.Cu) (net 8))
 (segment (start 84.408 101.092) (end 82.296 98.98) (width 0.3048) (layer B.Cu) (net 8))
 (segment (start 101.106 107.89) (end 99.762 107.89) (width 0.3048) (layer B.Cu) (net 9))
 (segment (start 99.762 107.89) (end 97.536 105.664) (width 0.3048) (layer B.Cu) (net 9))
 (segment (start 97.536 105.664) (end 97.536 101.346) (width 0.3048) (layer B.Cu) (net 9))
 (segment (start 94.742 98.552) (end 90.424 98.552) (width 0.3048) (layer B.Cu) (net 9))
 (segment (start 97.536 101.346) (end 94.742 98.552) (width 0.3048) (layer B.Cu) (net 9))
 (segment (start 90.424 98.552) (end 86.868 98.552) (width 0.3048) (layer B.Cu) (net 9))
 (segment (start 86.868 98.552) (end 82.296 93.98) (width 0.3048) (layer B.Cu) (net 9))
 (segment (start 83.646 128.27) (end 82.296 126.92) (width 0.3048) (layer B.Cu) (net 4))
 (segment (start 90.424 128.27) (end 83.646 128.27) (width 0.3048) (layer B.Cu) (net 4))
 (segment (start 90.424 128.27) (end 105.664 128.27) (width 0.3048) (layer F.Cu) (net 4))
 (segment (start 105.664 128.27) (end 115.824 118.11) (width 0.3048) (layer F.Cu) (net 4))
 (segment (start 115.824 118.11) (end 115.824 103.124) (width 0.3048) (layer F.Cu) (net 4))
 (segment (start 118.678 100.27) (end 121.506 100.27) (width 0.3048) (layer F.Cu) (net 4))
 (segment (start 115.824 103.124) (end 118.678 100.27) (width 0.3048) (layer F.Cu) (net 4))
 (segment (start 86.106 125.73) (end 82.296 121.92) (width 0.3048) (layer B.Cu) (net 5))
 (segment (start 90.424 125.73) (end 86.106 125.73) (width 0.3048) (layer B.Cu) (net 5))
 (segment (start 121.506 97.73) (end 119.44 97.73) (width 0.3048) (layer F.Cu) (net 5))
 (segment (start 119.44 97.73) (end 114.554 102.616) (width 0.3048) (layer F.Cu) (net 5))
 (segment (start 114.554 102.616) (end 114.554 117.602) (width 0.3048) (layer F.Cu) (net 5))
 (segment (start 114.554 117.602) (end 105.41 126.746) (width 0.3048) (layer F.Cu) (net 5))
 (segment (start 91.44 126.746) (end 90.424 125.73) (width 0.3048) (layer F.Cu) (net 5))
 (segment (start 105.41 126.746) (end 91.44 126.746) (width 0.3048) (layer F.Cu) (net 5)))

